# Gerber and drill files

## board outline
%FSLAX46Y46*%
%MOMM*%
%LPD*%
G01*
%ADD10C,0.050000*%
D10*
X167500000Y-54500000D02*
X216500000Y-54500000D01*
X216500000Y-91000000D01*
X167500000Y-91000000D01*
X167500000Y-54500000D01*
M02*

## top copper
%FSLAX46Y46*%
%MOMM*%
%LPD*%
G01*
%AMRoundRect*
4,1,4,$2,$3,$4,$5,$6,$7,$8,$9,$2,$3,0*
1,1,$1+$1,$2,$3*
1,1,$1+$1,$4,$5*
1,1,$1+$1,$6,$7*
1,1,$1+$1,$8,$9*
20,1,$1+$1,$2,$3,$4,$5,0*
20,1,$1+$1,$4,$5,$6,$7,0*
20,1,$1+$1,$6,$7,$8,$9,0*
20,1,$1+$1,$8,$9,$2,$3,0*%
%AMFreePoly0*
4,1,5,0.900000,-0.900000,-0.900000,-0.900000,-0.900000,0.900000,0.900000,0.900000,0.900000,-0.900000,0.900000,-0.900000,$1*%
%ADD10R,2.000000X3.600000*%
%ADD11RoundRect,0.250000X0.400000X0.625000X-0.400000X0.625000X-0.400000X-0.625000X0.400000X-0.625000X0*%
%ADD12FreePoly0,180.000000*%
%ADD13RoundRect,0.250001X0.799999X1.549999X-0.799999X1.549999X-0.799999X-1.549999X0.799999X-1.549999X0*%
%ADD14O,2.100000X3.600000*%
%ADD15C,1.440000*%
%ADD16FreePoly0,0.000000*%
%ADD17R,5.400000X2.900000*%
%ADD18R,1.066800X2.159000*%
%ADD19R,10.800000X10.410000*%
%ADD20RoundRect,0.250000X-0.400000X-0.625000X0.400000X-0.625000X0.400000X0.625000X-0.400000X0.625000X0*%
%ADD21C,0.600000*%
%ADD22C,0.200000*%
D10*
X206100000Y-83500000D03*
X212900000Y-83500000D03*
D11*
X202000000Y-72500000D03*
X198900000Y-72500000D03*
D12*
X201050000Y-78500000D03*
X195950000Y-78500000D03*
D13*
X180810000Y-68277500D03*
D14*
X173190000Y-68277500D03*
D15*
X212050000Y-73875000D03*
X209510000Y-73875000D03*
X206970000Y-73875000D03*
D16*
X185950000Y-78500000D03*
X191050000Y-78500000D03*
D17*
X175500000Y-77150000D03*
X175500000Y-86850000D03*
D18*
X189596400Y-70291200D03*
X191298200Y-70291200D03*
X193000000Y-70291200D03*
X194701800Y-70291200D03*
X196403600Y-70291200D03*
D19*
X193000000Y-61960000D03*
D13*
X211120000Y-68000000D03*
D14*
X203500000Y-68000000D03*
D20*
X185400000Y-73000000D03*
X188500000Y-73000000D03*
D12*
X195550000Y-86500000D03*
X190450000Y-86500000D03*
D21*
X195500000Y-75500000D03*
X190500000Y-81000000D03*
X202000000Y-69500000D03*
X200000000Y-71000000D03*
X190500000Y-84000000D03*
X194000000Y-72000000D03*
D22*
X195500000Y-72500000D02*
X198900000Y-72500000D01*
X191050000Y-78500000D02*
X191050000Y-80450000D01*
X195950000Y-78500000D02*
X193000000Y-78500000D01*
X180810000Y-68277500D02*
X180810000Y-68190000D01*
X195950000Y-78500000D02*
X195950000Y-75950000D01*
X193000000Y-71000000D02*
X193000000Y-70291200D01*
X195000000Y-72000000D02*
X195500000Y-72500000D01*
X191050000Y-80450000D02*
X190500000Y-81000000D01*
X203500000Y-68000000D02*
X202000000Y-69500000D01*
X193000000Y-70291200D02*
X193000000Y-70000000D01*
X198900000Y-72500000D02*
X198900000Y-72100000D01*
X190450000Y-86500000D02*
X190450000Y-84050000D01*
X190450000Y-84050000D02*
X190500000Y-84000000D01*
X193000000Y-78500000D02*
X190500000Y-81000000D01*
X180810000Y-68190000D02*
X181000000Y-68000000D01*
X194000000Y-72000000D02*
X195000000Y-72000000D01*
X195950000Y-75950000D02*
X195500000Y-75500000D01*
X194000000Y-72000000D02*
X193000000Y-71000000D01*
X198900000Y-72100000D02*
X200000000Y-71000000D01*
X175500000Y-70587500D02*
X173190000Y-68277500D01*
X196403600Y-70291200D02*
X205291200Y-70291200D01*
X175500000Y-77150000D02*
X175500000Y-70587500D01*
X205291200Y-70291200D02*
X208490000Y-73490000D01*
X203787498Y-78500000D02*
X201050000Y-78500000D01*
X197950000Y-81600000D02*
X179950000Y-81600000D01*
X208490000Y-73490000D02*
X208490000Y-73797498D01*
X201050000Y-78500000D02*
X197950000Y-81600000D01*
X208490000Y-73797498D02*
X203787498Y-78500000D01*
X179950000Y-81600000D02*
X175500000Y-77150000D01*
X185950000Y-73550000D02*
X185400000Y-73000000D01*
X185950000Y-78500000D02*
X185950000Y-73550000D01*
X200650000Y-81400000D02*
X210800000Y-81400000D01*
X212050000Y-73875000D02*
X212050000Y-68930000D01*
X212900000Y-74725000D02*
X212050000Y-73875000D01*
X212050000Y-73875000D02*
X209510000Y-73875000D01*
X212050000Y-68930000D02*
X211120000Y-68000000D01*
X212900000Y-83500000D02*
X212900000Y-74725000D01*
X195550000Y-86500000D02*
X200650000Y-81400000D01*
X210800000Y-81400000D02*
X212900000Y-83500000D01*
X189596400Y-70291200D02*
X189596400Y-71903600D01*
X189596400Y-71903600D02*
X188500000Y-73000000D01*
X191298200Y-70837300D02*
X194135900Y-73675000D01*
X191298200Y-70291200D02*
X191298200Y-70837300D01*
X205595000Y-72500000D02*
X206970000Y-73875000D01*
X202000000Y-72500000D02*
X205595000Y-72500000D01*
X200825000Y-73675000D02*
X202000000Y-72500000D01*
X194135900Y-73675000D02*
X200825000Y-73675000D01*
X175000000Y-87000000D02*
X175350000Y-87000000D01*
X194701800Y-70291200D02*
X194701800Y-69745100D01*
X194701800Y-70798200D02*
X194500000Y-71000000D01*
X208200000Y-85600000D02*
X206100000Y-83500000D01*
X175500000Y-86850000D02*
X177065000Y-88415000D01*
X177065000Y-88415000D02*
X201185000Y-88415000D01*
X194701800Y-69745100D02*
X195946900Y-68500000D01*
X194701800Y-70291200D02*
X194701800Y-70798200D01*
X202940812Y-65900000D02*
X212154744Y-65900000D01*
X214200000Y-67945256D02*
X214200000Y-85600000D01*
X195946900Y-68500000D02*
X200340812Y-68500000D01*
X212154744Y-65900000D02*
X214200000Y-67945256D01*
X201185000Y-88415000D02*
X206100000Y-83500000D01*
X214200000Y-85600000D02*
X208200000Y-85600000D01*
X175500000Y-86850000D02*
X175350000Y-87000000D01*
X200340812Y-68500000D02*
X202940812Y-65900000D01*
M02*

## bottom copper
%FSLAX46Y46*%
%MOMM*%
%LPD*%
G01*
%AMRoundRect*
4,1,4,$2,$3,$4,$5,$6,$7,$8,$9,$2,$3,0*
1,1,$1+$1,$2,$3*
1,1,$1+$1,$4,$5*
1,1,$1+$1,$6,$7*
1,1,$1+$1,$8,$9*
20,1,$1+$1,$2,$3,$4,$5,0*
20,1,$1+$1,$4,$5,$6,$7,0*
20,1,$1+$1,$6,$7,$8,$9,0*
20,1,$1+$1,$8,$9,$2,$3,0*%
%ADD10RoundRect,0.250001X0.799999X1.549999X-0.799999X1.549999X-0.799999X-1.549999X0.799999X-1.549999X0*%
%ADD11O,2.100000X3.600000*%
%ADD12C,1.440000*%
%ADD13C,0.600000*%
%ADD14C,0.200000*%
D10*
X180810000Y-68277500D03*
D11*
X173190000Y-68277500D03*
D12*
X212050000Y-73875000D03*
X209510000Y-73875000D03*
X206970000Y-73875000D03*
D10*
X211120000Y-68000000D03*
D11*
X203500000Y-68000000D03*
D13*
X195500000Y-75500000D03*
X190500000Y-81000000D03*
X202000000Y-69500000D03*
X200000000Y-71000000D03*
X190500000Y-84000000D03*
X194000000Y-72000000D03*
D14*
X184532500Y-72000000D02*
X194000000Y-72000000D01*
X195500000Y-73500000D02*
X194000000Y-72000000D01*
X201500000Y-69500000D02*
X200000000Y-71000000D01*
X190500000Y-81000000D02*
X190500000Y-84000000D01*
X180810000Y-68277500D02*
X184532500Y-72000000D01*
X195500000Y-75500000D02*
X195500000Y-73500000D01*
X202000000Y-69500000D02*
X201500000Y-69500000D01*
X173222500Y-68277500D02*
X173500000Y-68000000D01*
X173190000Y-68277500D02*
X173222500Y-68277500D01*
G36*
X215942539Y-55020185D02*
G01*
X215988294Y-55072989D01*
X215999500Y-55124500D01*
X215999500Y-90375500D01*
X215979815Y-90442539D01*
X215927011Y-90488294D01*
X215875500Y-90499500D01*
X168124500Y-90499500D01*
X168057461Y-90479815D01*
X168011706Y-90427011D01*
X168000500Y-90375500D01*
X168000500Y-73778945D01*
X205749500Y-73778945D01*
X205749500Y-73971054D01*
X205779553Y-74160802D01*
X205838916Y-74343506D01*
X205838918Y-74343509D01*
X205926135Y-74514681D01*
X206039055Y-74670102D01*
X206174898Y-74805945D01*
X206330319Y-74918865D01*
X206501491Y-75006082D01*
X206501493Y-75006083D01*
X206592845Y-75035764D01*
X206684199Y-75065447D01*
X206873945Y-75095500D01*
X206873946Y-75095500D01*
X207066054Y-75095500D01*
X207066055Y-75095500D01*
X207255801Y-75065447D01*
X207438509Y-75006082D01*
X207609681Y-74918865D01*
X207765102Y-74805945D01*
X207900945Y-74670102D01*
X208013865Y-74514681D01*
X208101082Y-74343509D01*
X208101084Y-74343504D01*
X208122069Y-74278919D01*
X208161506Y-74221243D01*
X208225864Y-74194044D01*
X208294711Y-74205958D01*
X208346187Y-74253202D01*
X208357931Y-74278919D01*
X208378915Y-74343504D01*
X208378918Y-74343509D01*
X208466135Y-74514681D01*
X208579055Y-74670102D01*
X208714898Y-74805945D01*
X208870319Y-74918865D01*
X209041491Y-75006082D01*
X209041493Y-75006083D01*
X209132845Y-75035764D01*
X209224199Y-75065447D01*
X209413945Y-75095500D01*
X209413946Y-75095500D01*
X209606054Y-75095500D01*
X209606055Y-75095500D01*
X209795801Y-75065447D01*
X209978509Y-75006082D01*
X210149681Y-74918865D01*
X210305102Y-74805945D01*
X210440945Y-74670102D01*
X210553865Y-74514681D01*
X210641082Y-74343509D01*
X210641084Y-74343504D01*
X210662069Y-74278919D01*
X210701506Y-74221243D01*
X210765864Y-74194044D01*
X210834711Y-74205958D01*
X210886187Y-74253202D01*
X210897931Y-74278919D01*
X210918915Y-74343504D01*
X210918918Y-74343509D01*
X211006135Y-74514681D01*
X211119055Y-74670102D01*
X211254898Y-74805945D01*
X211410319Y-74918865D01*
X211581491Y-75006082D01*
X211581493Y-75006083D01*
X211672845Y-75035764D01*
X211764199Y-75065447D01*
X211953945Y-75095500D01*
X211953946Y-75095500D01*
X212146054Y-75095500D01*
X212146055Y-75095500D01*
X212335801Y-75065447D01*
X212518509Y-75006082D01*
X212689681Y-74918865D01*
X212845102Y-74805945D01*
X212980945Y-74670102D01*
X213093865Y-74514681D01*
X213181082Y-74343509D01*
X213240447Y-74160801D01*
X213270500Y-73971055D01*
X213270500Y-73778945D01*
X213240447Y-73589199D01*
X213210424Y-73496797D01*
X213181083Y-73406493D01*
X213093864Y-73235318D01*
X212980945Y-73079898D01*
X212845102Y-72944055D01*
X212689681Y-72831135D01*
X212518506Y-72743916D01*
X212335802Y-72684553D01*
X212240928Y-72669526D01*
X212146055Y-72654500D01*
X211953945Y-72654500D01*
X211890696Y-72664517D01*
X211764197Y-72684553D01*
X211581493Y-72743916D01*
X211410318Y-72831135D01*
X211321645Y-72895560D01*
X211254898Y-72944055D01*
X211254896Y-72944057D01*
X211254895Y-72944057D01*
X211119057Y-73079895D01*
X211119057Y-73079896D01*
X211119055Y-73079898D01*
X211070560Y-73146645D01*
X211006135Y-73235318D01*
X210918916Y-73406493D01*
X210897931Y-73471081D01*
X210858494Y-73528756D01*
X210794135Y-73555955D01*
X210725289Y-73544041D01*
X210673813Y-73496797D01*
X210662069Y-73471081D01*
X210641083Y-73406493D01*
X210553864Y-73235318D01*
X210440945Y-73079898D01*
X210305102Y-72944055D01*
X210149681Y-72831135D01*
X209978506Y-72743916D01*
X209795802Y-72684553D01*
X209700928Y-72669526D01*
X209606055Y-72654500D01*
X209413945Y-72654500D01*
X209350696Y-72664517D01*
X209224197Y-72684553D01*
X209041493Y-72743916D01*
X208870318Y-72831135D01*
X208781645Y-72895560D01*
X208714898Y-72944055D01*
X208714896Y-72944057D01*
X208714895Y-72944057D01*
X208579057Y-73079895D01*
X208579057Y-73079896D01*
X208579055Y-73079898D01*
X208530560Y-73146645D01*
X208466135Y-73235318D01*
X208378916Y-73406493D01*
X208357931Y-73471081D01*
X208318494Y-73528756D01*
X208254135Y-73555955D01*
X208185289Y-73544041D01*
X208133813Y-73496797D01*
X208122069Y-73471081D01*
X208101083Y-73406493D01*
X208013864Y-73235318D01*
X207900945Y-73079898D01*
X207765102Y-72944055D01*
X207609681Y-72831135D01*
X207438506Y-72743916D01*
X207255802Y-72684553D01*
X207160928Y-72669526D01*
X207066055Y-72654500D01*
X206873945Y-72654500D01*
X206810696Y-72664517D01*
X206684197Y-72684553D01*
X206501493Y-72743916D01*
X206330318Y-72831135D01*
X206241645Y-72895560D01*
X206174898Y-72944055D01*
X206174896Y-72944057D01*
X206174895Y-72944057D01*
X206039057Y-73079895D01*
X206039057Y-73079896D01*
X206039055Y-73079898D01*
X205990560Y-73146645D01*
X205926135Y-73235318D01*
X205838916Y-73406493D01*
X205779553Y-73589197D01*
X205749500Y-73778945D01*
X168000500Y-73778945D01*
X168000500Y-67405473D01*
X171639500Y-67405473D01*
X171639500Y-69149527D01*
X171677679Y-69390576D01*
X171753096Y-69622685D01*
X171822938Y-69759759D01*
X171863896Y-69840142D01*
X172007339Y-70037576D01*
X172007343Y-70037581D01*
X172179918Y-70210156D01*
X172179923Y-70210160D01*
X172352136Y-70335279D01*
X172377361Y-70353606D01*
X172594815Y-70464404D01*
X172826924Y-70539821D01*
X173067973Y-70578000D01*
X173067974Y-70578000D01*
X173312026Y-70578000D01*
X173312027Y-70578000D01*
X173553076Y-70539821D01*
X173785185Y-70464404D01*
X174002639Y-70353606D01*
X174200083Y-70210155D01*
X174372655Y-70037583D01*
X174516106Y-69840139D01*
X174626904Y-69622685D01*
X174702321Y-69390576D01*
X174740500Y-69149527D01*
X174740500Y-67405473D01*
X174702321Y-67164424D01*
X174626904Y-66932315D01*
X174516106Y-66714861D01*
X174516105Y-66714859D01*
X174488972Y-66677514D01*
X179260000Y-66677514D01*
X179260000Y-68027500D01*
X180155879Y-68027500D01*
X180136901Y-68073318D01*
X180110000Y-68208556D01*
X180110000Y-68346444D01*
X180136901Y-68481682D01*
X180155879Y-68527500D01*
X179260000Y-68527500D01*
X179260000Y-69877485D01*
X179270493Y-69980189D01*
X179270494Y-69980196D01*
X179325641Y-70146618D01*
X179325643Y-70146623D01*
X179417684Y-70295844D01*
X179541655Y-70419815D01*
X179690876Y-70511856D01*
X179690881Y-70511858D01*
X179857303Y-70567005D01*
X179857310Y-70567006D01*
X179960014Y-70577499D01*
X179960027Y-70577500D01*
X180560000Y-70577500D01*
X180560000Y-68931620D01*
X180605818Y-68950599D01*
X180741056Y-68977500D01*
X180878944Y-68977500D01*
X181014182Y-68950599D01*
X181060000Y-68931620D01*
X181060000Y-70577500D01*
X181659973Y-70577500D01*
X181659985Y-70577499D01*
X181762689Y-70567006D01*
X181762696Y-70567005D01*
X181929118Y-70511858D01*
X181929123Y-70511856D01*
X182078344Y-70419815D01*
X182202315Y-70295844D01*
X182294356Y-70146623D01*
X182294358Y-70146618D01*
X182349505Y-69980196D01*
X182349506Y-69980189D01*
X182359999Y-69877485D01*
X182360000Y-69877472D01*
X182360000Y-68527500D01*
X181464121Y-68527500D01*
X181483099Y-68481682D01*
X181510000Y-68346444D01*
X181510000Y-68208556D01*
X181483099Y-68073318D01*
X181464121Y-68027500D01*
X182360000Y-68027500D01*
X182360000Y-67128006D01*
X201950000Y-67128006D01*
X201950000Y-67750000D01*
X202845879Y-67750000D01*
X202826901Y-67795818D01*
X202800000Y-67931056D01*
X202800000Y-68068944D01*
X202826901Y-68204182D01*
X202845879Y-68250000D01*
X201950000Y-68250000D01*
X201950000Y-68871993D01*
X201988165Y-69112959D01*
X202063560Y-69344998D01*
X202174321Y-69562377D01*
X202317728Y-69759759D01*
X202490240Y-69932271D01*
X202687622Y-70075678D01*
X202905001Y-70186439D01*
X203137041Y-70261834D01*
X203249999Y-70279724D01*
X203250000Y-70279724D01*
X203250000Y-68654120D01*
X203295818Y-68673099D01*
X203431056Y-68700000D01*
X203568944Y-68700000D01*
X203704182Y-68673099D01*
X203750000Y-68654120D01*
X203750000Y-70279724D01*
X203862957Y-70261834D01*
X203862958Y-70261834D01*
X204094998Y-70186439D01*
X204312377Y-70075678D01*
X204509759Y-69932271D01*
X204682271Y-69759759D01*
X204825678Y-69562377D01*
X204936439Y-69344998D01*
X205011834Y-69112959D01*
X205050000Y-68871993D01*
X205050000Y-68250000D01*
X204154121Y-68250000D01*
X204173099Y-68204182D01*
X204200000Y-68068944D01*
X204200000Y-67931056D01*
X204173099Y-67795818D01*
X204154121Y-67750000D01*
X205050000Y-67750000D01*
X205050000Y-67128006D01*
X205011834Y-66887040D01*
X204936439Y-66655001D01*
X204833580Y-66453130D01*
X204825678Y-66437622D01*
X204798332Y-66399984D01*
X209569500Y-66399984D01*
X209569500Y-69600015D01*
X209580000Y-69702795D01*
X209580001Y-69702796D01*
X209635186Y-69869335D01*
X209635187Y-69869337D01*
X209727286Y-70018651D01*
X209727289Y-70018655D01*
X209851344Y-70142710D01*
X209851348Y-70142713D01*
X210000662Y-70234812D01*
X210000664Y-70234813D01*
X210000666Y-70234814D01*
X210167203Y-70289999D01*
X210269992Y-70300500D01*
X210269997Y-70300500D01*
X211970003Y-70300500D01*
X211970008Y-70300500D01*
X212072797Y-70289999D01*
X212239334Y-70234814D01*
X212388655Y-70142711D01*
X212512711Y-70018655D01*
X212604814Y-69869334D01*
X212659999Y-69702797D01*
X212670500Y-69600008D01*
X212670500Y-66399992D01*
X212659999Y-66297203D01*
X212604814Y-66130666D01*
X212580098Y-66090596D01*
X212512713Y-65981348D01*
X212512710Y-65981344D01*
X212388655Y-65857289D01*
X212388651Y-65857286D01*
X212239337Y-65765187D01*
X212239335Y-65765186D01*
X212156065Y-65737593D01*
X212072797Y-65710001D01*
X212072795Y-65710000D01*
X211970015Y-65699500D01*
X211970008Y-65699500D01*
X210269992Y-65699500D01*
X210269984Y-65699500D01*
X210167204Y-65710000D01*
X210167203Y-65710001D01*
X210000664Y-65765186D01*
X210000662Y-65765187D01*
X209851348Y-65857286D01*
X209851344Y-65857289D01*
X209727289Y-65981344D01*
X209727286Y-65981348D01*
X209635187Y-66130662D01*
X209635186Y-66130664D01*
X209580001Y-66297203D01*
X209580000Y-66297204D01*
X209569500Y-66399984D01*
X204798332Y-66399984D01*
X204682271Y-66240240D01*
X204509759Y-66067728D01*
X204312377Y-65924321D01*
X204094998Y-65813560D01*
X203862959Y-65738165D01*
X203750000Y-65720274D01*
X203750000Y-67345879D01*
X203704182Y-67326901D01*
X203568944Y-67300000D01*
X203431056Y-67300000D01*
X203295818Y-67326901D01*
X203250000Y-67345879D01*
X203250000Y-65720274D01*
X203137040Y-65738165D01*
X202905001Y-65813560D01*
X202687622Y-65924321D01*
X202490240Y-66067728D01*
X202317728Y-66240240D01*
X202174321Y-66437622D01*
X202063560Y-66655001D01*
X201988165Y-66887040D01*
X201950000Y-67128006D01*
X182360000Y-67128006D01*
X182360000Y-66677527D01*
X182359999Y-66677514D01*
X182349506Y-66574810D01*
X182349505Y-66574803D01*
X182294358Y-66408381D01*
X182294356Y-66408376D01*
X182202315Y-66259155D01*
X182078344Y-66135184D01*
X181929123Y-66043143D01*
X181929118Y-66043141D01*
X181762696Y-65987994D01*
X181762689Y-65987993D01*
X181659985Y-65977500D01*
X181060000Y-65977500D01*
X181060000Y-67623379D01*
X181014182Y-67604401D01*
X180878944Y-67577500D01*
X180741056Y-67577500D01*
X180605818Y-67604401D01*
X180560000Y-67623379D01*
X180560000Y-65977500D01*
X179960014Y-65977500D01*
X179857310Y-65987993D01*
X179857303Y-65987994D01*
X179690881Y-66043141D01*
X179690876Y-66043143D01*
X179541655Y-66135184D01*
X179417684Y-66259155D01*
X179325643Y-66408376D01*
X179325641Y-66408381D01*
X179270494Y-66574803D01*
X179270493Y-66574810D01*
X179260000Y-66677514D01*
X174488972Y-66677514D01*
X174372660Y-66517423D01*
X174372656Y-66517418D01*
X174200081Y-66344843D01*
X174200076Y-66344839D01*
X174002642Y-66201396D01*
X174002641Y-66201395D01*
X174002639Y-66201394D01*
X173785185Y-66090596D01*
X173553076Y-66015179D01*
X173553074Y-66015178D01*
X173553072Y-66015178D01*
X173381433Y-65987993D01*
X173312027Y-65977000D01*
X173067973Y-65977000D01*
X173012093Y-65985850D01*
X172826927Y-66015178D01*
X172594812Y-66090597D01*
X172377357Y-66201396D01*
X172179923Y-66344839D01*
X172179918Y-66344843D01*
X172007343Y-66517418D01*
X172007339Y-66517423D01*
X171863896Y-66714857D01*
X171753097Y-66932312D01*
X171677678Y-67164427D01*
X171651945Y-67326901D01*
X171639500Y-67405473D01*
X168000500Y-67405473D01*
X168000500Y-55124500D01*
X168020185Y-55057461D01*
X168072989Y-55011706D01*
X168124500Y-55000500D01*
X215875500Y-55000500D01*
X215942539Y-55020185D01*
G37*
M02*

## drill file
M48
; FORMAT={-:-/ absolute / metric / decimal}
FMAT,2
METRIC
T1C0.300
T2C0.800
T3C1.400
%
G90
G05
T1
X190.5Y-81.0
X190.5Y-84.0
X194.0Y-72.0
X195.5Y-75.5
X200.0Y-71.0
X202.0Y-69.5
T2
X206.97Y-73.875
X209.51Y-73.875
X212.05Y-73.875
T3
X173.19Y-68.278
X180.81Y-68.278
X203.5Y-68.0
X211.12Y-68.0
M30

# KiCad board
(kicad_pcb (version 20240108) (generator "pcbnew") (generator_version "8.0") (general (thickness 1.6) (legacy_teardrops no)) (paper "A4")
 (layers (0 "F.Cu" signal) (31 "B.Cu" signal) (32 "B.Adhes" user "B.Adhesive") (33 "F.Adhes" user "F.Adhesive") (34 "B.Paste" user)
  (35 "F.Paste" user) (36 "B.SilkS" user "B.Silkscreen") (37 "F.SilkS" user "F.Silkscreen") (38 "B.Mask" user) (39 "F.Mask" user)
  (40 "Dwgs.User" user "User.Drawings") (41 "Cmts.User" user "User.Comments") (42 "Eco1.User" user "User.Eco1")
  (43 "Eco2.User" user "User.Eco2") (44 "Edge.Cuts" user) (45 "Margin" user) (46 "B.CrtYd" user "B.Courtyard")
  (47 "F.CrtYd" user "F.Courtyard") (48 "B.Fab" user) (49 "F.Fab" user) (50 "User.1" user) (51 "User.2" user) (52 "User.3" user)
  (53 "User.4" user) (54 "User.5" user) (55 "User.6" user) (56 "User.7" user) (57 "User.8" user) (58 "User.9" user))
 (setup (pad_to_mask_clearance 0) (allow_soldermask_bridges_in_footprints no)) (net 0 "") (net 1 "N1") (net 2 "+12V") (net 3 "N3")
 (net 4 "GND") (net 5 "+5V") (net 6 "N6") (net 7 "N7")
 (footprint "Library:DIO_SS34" (layer "F.Cu") (at 209.5 83.5 180)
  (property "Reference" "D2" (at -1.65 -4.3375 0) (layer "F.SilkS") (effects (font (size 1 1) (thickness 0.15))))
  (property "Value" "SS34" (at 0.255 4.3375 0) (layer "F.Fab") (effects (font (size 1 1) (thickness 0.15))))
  (pad "A" smd rect (at 3.4 0 180) (size 2 3.6) (layers "F.Cu" "F.Paste" "F.Mask") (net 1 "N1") (solder_mask_margin 0.102))
  (pad "C" smd rect (at -3.4 0 180) (size 2 3.6) (layers "F.Cu" "F.Paste" "F.Mask") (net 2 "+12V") (solder_mask_margin 0.102)))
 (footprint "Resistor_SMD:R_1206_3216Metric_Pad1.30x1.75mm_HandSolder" (layer "F.Cu") (at 200.45 72.5 180)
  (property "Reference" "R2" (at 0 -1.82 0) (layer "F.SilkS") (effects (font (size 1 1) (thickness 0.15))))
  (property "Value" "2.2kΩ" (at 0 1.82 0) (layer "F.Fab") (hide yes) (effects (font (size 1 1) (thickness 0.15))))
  (pad "1" smd roundrect (at -1.55 0 180) (size 1.3 1.75) (layers "F.Cu" "F.Paste" "F.Mask") (roundrect_rratio 0.192308) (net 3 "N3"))
  (pad "2" smd roundrect (at 1.55 0 180) (size 1.3 1.75) (layers "F.Cu" "F.Paste" "F.Mask") (roundrect_rratio 0.192308) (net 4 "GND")))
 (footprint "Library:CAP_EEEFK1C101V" (layer "F.Cu") (at 198.5 78.5 180)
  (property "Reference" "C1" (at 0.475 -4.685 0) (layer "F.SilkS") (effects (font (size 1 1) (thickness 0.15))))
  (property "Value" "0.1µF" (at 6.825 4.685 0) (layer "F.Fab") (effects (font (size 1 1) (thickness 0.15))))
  (pad "1" smd custom (at -2.55 0 180) (size 1.8 1.8) (layers "F.Cu") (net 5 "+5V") (options (clearance outline) (anchor rect)) (primitives))
  (pad "2" smd custom (at 2.55 0 180) (size 1.8 1.8) (layers "F.Cu") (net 4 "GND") (options (clearance outline) (anchor rect)) (primitives)))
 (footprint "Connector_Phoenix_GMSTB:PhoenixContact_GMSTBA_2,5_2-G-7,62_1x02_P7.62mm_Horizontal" (layer "F.Cu") (at 180.81 68.2775 180)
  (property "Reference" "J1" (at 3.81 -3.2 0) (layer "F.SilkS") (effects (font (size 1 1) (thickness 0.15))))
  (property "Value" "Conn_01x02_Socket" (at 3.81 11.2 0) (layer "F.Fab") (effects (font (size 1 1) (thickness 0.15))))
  (pad "1" thru_hole roundrect (at 0 0 180) (size 2.1 3.6) (drill 1.4) (layers "*.Cu" "*.Mask") (remove_unused_layers no)
   (roundrect_rratio 0.119048) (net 4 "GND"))
  (pad "2" thru_hole oval (at 7.62 0 180) (size 2.1 3.6) (drill 1.4) (layers "*.Cu" "*.Mask") (remove_unused_layers no) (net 5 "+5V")))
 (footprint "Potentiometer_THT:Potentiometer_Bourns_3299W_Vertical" (layer "F.Cu") (at 212.05 73.875)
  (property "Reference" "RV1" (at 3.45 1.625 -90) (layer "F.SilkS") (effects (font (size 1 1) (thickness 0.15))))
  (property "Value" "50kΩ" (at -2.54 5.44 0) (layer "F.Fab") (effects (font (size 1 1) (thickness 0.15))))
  (pad "1" thru_hole circle (at 0 0) (size 1.44 1.44) (drill 0.8) (layers "*.Cu" "*.Mask") (remove_unused_layers no) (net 2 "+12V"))
  (pad "2" thru_hole circle (at -2.54 0) (size 1.44 1.44) (drill 0.8) (layers "*.Cu" "*.Mask") (remove_unused_layers no) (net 2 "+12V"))
  (pad "3" thru_hole circle (at -5.08 0) (size 1.44 1.44) (drill 0.8) (layers "*.Cu" "*.Mask") (remove_unused_layers no) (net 3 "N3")))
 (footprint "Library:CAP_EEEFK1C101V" (layer "F.Cu") (at 188.5 78.5)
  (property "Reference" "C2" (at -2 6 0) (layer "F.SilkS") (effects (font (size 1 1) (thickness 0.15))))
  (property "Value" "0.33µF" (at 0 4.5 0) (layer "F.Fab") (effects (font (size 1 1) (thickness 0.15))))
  (pad "1" smd custom (at -2.55 0) (size 1.8 1.8) (layers "F.Cu") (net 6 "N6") (options (clearance outline) (anchor rect)) (primitives))
  (pad "2" smd custom (at 2.55 0) (size 1.8 1.8) (layers "F.Cu") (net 4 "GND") (options (clearance outline) (anchor rect)) (primitives)))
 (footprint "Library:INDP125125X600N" (layer "F.Cu") (at 175.5 82 -90)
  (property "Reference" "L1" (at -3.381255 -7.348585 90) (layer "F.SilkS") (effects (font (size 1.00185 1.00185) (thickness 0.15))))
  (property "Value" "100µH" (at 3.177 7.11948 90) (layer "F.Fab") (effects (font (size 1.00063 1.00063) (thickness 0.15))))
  (pad "1" smd rect (at -4.85 0 270) (size 2.9 5.4) (layers "F.Cu" "F.Paste" "F.Mask") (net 5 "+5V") (solder_mask_margin 0.102))
  (pad "2" smd rect (at 4.85 0 270) (size 2.9 5.4) (layers "F.Cu" "F.Paste" "F.Mask") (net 1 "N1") (solder_mask_margin 0.102)))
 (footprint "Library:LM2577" (layer "F.Cu") (at 193 64.5)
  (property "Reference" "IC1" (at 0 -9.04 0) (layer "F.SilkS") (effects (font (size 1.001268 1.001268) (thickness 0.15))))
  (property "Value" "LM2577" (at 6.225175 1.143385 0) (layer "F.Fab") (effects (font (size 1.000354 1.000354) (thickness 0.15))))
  (pad "1" smd rect (at -3.4036 5.7912) (size 1.0668 2.159) (layers "F.Cu" "F.Paste" "F.Mask") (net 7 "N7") (solder_mask_margin 0.102))
  (pad "2" smd rect (at -1.7018 5.7912) (size 1.0668 2.159) (layers "F.Cu" "F.Paste" "F.Mask") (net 3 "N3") (solder_mask_margin 0.102))
  (pad "3" smd rect (at 0 5.7912) (size 1.0668 2.159) (layers "F.Cu" "F.Paste" "F.Mask") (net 4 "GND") (solder_mask_margin 0.102))
  (pad "4" smd rect (at 1.7018 5.7912) (size 1.0668 2.159) (layers "F.Cu" "F.Paste" "F.Mask") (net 1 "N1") (solder_mask_margin 0.102))
  (pad "5" smd rect (at 3.4036 5.7912) (size 1.0668 2.159) (layers "F.Cu" "F.Paste" "F.Mask") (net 5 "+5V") (solder_mask_margin 0.102))
  (pad "6" smd rect (at 0 -2.54) (size 10.8 10.41) (layers "F.Cu" "F.Paste" "F.Mask") (solder_mask_margin 0.102)))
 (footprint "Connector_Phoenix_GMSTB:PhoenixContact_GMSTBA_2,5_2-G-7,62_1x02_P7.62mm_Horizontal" (layer "F.Cu") (at 211.12 68 180)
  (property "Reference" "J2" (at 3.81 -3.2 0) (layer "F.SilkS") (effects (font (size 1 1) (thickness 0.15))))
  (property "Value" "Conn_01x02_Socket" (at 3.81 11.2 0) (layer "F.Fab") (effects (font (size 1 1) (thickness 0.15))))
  (pad "1" thru_hole roundrect (at 0 0 180) (size 2.1 3.6) (drill 1.4) (layers "*.Cu" "*.Mask") (remove_unused_layers no)
   (roundrect_rratio 0.119048) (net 2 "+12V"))
  (pad "2" thru_hole oval (at 7.62 0 180) (size 2.1 3.6) (drill 1.4) (layers "*.Cu" "*.Mask") (remove_unused_layers no) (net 4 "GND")))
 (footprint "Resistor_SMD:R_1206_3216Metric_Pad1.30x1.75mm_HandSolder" (layer "F.Cu") (at 186.95 73)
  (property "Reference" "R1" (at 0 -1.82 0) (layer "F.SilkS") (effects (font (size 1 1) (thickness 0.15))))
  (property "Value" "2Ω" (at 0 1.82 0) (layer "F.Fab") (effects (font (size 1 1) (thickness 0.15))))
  (pad "1" smd roundrect (at -1.55 0) (size 1.3 1.75) (layers "F.Cu" "F.Paste" "F.Mask") (roundrect_rratio 0.192308) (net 6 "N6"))
  (pad "2" smd roundrect (at 1.55 0) (size 1.3 1.75) (layers "F.Cu" "F.Paste" "F.Mask") (roundrect_rratio 0.192308) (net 7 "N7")))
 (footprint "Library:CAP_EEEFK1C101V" (layer "F.Cu") (at 193 86.5 180)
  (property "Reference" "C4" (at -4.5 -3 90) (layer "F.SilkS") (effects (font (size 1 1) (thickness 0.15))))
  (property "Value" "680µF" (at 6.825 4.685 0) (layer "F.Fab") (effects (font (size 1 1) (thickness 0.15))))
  (pad "1" smd custom (at -2.55 0 180) (size 1.8 1.8) (layers "F.Cu") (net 2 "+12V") (options (clearance outline) (anchor rect))
   (primitives))
  (pad "2" smd custom (at 2.55 0 180) (size 1.8 1.8) (layers "F.Cu") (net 4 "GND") (options (clearance outline) (anchor rect)) (primitives)))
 (gr_rect (start 167.5 54.5) (end 216.5 91) (stroke (width 0.05) (type default)) (fill none) (layer "Edge.Cuts"))
 (segment (start 195.5 72.5) (end 198.9 72.5) (width 0.2) (layer "F.Cu") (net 4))
 (segment (start 191.05 78.5) (end 191.05 80.45) (width 0.2) (layer "F.Cu") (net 4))
 (segment (start 195.95 78.5) (end 193 78.5) (width 0.2) (layer "F.Cu") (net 4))
 (segment (start 180.81 68.2775) (end 180.81 68.19) (width 0.2) (layer "F.Cu") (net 4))
 (segment (start 195.95 78.5) (end 195.95 75.95) (width 0.2) (layer "F.Cu") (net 4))
 (segment (start 193 71) (end 193 70.2912) (width 0.2) (layer "F.Cu") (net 4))
 (segment (start 195 72) (end 195.5 72.5) (width 0.2) (layer "F.Cu") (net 4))
 (segment (start 191.05 80.45) (end 190.5 81) (width 0.2) (layer "F.Cu") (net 4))
 (segment (start 203.5 68) (end 202 69.5) (width 0.2) (layer "F.Cu") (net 4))
 (segment (start 193 70.2912) (end 193 70) (width 0.2) (layer "F.Cu") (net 4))
 (segment (start 198.9 72.5) (end 198.9 72.1) (width 0.2) (layer "F.Cu") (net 4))
 (segment (start 190.45 86.5) (end 190.45 84.05) (width 0.2) (layer "F.Cu") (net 4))
 (segment (start 190.45 84.05) (end 190.5 84) (width 0.2) (layer "F.Cu") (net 4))
 (segment (start 193 78.5) (end 190.5 81) (width 0.2) (layer "F.Cu") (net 4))
 (segment (start 180.81 68.19) (end 181 68) (width 0.2) (layer "F.Cu") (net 4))
 (segment (start 194 72) (end 195 72) (width 0.2) (layer "F.Cu") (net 4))
 (segment (start 195.95 75.95) (end 195.5 75.5) (width 0.2) (layer "F.Cu") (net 4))
 (segment (start 194 72) (end 193 71) (width 0.2) (layer "F.Cu") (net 4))
 (segment (start 198.9 72.1) (end 200 71) (width 0.2) (layer "F.Cu") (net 4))
 (via (at 195.5 75.5) (size 0.6) (drill 0.3) (layers "F.Cu" "B.Cu") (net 4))
 (via (at 190.5 81) (size 0.6) (drill 0.3) (layers "F.Cu" "B.Cu") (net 4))
 (via (at 202 69.5) (size 0.6) (drill 0.3) (layers "F.Cu" "B.Cu") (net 4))
 (via (at 200 71) (size 0.6) (drill 0.3) (layers "F.Cu" "B.Cu") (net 4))
 (via (at 190.5 84) (size 0.6) (drill 0.3) (layers "F.Cu" "B.Cu") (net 4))
 (via (at 194 72) (size 0.6) (drill 0.3) (layers "F.Cu" "B.Cu") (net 4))
 (segment (start 184.5325 72) (end 194 72) (width 0.2) (layer "B.Cu") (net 4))
 (segment (start 195.5 73.5) (end 194 72) (width 0.2) (layer "B.Cu") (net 4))
 (segment (start 201.5 69.5) (end 200 71) (width 0.2) (layer "B.Cu") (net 4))
 (segment (start 190.5 81) (end 190.5 84) (width 0.2) (layer "B.Cu") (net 4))
 (segment (start 180.81 68.2775) (end 184.5325 72) (width 0.2) (layer "B.Cu") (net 4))
 (segment (start 195.5 75.5) (end 195.5 73.5) (width 0.2) (layer "B.Cu") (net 4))
 (segment (start 202 69.5) (end 201.5 69.5) (width 0.2) (layer "B.Cu") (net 4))
 (segment (start 175.5 70.5875) (end 173.19 68.2775) (width 0.2) (layer "F.Cu") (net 5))
 (segment (start 196.4036 70.2912) (end 205.2912 70.2912) (width 0.2) (layer "F.Cu") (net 5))
 (segment (start 175.5 77.15) (end 175.5 70.5875) (width 0.2) (layer "F.Cu") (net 5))
 (segment (start 205.2912 70.2912) (end 208.49 73.49) (width 0.2) (layer "F.Cu") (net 5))
 (segment (start 203.787498 78.5) (end 201.05 78.5) (width 0.2) (layer "F.Cu") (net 5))
 (segment (start 197.95 81.6) (end 179.95 81.6) (width 0.2) (layer "F.Cu") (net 5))
 (segment (start 208.49 73.49) (end 208.49 73.797498) (width 0.2) (layer "F.Cu") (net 5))
 (segment (start 201.05 78.5) (end 197.95 81.6) (width 0.2) (layer "F.Cu") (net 5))
 (segment (start 208.49 73.797498) (end 203.787498 78.5) (width 0.2) (layer "F.Cu") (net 5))
 (segment (start 179.95 81.6) (end 175.5 77.15) (width 0.2) (layer "F.Cu") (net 5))
 (segment (start 173.2225 68.2775) (end 173.5 68) (width 0.2) (layer "B.Cu") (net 5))
 (segment (start 173.19 68.2775) (end 173.2225 68.2775) (width 0.2) (layer "B.Cu") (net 5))
 (segment (start 185.95 73.55) (end 185.4 73) (width 0.2) (layer "F.Cu") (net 6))
 (segment (start 185.95 78.5) (end 185.95 73.55) (width 0.2) (layer "F.Cu") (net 6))
 (segment (start 200.65 81.4) (end 210.8 81.4) (width 0.2) (layer "F.Cu") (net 2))
 (segment (start 212.05 73.875) (end 212.05 68.93) (width 0.2) (layer "F.Cu") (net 2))
 (segment (start 212.9 74.725) (end 212.05 73.875) (width 0.2) (layer "F.Cu") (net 2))
 (segment (start 212.05 73.875) (end 209.51 73.875) (width 0.2) (layer "F.Cu") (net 2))
 (segment (start 212.05 68.93) (end 211.12 68) (width 0.2) (layer "F.Cu") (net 2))
 (segment (start 212.9 83.5) (end 212.9 74.725) (width 0.2) (layer "F.Cu") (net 2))
 (segment (start 195.55 86.5) (end 200.65 81.4) (width 0.2) (layer "F.Cu") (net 2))
 (segment (start 210.8 81.4) (end 212.9 83.5) (width 0.2) (layer "F.Cu") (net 2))
 (segment (start 189.5964 70.2912) (end 189.5964 71.9036) (width 0.2) (layer "F.Cu") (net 7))
 (segment (start 189.5964 71.9036) (end 188.5 73) (width 0.2) (layer "F.Cu") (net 7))
 (segment (start 191.2982 70.8373) (end 194.1359 73.675) (width 0.2) (layer "F.Cu") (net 3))
 (segment (start 191.2982 70.2912) (end 191.2982 70.8373) (width 0.2) (layer "F.Cu") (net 3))
 (segment (start 205.595 72.5) (end 206.97 73.875) (width 0.2) (layer "F.Cu") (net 3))
 (segment (start 202 72.5) (end 205.595 72.5) (width 0.2) (layer "F.Cu") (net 3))
 (segment (start 200.825 73.675) (end 202 72.5) (width 0.2) (layer "F.Cu") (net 3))
 (segment (start 194.1359 73.675) (end 200.825 73.675) (width 0.2) (layer "F.Cu") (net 3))
 (segment (start 175 87) (end 175.35 87) (width 0.2) (layer "F.Cu") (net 1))
 (segment (start 194.7018 70.2912) (end 194.7018 69.7451) (width 0.2) (layer "F.Cu") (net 1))
 (segment (start 194.7018 70.7982) (end 194.5 71) (width 0.2) (layer "F.Cu") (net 1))
 (segment (start 208.2 85.6) (end 206.1 83.5) (width 0.2) (layer "F.Cu") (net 1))
 (segment (start 175.5 86.85) (end 177.065 88.415) (width 0.2) (layer "F.Cu") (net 1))
 (segment (start 177.065 88.415) (end 201.185 88.415) (width 0.2) (layer "F.Cu") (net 1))
 (segment (start 194.7018 69.7451) (end 195.9469 68.5) (width 0.2) (layer "F.Cu") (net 1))
 (segment (start 194.7018 70.2912) (end 194.7018 70.7982) (width 0.2) (layer "F.Cu") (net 1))
 (segment (start 202.940812 65.9) (end 212.154744 65.9) (width 0.2) (layer "F.Cu") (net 1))
 (segment (start 214.2 67.945256) (end 214.2 85.6) (width 0.2) (layer "F.Cu") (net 1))
 (segment (start 195.9469 68.5) (end 200.340812 68.5) (width 0.2) (layer "F.Cu") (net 1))
 (segment (start 212.154744 65.9) (end 214.2 67.945256) (width 0.2) (layer "F.Cu") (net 1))
 (segment (start 201.185 88.415) (end 206.1 83.5) (width 0.2) (layer "F.Cu") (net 1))
 (segment (start 214.2 85.6) (end 208.2 85.6) (width 0.2) (layer "F.Cu") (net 1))
 (segment (start 175.5 86.85) (end 175.35 87) (width 0.2) (layer "F.Cu") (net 1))
 (segment (start 200.340812 68.5) (end 202.940812 65.9) (width 0.2) (layer "F.Cu") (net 1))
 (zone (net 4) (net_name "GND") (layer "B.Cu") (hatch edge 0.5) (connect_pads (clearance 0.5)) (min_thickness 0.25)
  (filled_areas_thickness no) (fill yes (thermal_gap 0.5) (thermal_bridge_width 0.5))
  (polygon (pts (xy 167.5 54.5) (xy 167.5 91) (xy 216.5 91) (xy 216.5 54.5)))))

